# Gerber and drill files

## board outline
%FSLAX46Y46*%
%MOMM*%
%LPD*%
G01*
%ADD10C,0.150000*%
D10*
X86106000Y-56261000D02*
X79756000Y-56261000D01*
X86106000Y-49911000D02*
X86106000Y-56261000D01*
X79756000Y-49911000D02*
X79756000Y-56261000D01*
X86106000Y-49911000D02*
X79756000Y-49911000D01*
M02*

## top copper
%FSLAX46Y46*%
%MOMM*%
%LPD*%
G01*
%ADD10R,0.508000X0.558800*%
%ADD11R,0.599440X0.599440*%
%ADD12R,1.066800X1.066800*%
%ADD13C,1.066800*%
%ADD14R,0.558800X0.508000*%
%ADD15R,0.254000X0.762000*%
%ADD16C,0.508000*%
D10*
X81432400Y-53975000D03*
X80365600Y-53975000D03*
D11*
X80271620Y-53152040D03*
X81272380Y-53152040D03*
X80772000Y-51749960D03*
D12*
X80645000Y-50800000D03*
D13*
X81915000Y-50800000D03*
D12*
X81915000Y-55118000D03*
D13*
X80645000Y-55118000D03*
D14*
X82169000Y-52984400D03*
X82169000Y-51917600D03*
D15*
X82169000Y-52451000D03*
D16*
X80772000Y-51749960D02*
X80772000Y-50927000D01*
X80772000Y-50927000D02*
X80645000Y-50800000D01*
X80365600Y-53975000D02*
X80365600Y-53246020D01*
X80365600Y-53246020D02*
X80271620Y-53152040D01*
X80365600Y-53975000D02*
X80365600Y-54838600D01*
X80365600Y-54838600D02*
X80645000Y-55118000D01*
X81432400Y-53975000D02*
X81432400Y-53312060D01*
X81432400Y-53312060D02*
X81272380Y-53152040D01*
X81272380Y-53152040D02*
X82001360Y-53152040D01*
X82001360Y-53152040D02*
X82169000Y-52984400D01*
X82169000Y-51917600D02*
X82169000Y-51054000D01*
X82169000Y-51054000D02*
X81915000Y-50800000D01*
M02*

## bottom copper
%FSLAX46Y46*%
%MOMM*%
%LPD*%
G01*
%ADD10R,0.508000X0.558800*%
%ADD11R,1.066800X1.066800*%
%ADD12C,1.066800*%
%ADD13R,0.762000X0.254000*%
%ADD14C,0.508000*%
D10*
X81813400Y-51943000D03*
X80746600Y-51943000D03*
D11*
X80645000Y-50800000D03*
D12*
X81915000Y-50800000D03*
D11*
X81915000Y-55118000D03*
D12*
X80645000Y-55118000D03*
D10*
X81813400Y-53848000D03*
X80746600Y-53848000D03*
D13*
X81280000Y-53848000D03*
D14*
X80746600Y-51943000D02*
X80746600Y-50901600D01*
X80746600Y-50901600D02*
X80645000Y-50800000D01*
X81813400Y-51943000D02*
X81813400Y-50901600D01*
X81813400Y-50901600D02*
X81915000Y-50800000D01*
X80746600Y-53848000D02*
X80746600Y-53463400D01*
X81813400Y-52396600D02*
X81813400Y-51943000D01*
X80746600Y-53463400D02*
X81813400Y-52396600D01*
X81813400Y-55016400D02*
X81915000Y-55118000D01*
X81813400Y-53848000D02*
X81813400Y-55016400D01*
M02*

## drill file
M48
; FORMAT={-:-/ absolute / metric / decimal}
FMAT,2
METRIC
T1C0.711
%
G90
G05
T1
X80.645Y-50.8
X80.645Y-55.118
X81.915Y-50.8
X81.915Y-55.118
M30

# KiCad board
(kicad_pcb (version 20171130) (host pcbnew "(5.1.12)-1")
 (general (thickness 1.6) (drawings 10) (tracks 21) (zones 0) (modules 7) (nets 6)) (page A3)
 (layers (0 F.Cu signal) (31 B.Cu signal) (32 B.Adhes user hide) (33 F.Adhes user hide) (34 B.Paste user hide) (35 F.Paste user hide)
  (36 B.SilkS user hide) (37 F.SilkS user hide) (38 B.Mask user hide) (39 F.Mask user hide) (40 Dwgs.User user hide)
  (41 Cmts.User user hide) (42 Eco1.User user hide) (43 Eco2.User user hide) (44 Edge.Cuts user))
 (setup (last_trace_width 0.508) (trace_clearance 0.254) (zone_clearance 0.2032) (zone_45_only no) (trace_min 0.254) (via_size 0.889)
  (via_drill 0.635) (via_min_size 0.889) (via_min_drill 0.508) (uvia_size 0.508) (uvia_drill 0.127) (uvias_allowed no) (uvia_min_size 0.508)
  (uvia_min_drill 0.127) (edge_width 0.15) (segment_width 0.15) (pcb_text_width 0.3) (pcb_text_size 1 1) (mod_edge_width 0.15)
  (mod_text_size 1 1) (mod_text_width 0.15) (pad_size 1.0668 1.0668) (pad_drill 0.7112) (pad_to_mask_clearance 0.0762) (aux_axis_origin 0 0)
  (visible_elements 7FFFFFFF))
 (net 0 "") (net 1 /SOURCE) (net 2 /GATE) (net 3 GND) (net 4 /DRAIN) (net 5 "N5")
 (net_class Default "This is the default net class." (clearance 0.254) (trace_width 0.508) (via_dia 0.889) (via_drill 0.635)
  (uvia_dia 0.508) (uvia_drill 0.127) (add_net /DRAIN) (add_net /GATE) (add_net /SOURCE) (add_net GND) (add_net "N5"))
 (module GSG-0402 (layer F.Cu) (at 80.899 53.975) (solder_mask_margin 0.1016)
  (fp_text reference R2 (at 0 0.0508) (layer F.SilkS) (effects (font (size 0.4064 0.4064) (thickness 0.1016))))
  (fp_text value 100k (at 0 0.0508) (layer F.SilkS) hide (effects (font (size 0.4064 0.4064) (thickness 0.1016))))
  (pad 2 smd rect (at 0.5334 0) (size 0.508 0.5588) (layers F.Cu F.Paste F.Mask) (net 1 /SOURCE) (solder_mask_margin 0.1016))
  (pad 1 smd rect (at -0.5334 0) (size 0.508 0.5588) (layers F.Cu F.Paste F.Mask) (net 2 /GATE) (die_length -1518.485687)
   (solder_mask_margin 0.1016)))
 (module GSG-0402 (layer B.Cu) (at 81.28 51.943) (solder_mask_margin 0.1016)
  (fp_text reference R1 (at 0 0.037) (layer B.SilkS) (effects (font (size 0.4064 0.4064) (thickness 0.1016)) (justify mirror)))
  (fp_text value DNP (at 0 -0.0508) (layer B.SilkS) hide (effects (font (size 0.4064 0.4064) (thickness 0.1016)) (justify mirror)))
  (pad 2 smd rect (at 0.5334 0) (size 0.508 0.5588) (layers B.Cu B.Paste B.Mask) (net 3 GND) (solder_mask_margin 0.1016))
  (pad 1 smd rect (at -0.5334 0) (size 0.508 0.5588) (layers B.Cu B.Paste B.Mask) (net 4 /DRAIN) (die_length -1518.485687)
   (solder_mask_margin 0.1016)))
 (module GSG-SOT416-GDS (layer F.Cu) (at 80.772 52.451)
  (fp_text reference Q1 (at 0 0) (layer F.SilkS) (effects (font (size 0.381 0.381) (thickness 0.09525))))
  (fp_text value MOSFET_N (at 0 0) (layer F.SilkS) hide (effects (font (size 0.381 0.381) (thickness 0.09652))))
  (pad G smd rect (at -0.50038 0.70104) (size 0.59944 0.59944) (layers F.Cu F.Paste F.Mask) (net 2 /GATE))
  (pad S smd rect (at 0.50038 0.70104) (size 0.59944 0.59944) (layers F.Cu F.Paste F.Mask) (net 1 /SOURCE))
  (pad D smd rect (at 0 -0.70104) (size 0.59944 0.59944) (layers F.Cu F.Paste F.Mask) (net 4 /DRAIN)))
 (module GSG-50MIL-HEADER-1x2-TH (layer F.Cu) (at 81.28 50.8)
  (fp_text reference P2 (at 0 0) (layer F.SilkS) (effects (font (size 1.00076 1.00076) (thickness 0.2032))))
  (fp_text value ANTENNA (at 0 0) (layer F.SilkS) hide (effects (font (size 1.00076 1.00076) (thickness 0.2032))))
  (pad 1 thru_hole rect (at -0.635 0) (size 1.0668 1.0668) (drill 0.7112) (layers *.Cu *.Mask) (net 4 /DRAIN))
  (pad 2 thru_hole circle (at 0.635 0) (size 1.0668 1.0668) (drill 0.7112) (layers *.Cu *.Mask) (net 3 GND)))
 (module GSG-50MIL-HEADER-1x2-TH (layer F.Cu) (at 81.28 55.118 180)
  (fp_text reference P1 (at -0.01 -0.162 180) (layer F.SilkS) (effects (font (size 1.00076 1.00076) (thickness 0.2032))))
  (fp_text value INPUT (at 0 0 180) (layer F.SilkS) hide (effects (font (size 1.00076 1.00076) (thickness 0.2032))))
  (pad 1 thru_hole rect (at -0.635 0 180) (size 1.0668 1.0668) (drill 0.7112) (layers *.Cu *.Mask) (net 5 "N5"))
  (pad 2 thru_hole circle (at 0.635 0 180) (size 1.0668 1.0668) (drill 0.7112) (layers *.Cu *.Mask) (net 2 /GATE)))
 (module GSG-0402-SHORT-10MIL (layer B.Cu) (at 81.28 53.848) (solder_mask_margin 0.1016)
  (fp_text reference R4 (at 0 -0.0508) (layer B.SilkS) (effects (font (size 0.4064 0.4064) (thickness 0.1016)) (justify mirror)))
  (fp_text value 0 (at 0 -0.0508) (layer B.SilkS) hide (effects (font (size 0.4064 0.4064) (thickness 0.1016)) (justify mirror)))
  (pad 2 smd rect (at 0.5334 0) (size 0.508 0.5588) (layers B.Cu B.Mask) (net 5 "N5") (solder_mask_margin 0.1016))
  (pad 1 smd rect (at -0.5334 0) (size 0.508 0.5588) (layers B.Cu B.Mask) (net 3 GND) (die_length -1518.485687) (solder_mask_margin 0.1016))
  (pad "" smd rect (at 0 0) (size 0.762 0.254) (layers B.Cu B.Mask)))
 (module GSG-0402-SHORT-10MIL (layer F.Cu) (at 82.169 52.451 270) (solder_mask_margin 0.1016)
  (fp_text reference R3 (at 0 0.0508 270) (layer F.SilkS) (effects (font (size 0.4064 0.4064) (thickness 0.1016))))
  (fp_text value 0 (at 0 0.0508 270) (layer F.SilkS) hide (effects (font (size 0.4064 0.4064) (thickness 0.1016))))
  (pad 2 smd rect (at 0.5334 0 270) (size 0.508 0.5588) (layers F.Cu F.Mask) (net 1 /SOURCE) (solder_mask_margin 0.1016))
  (pad 1 smd rect (at -0.5334 0 270) (size 0.508 0.5588) (layers F.Cu F.Mask) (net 3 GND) (die_length -1518.485687)
   (solder_mask_margin 0.1016))
  (pad "" smd rect (at 0 0 270) (size 0.762 0.254) (layers F.Cu F.Mask)))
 (gr_line (start 86.106 56.261) (end 79.756 56.261) (angle 90) (layer Edge.Cuts) (width 0.15))
 (gr_line (start 86.106 49.911) (end 86.106 56.261) (angle 90) (layer Edge.Cuts) (width 0.15))
 (gr_line (start 79.756 49.911) (end 79.756 56.261) (angle 90) (layer Edge.Cuts) (width 0.15))
 (gr_line (start 86.106 49.911) (end 79.756 49.911) (angle 90) (layer Edge.Cuts) (width 0.15))
 (segment (start 80.7466 51.943) (end 80.7466 50.9016) (width 0.508) (layer B.Cu) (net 4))
 (segment (start 80.7466 50.9016) (end 80.645 50.8) (width 0.508) (layer B.Cu) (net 4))
 (segment (start 80.772 51.74996) (end 80.772 50.927) (width 0.508) (layer F.Cu) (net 4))
 (segment (start 80.772 50.927) (end 80.645 50.8) (width 0.508) (layer F.Cu) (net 4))
 (segment (start 80.3656 53.975) (end 80.3656 53.24602) (width 0.508) (layer F.Cu) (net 2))
 (segment (start 80.3656 53.24602) (end 80.27162 53.15204) (width 0.508) (layer F.Cu) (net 2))
 (segment (start 80.3656 53.975) (end 80.3656 54.8386) (width 0.508) (layer F.Cu) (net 2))
 (segment (start 80.3656 54.8386) (end 80.645 55.118) (width 0.508) (layer F.Cu) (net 2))
 (segment (start 81.4324 53.975) (end 81.4324 53.31206) (width 0.508) (layer F.Cu) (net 1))
 (segment (start 81.4324 53.31206) (end 81.27238 53.15204) (width 0.508) (layer F.Cu) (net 1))
 (segment (start 81.27238 53.15204) (end 82.00136 53.15204) (width 0.508) (layer F.Cu) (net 1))
 (segment (start 82.00136 53.15204) (end 82.169 52.9844) (width 0.508) (layer F.Cu) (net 1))
 (segment (start 81.8134 51.943) (end 81.8134 50.9016) (width 0.508) (layer B.Cu) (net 3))
 (segment (start 81.8134 50.9016) (end 81.915 50.8) (width 0.508) (layer B.Cu) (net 3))
 (segment (start 80.7466 53.848) (end 80.7466 53.4634) (width 0.508) (layer B.Cu) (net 3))
 (segment (start 81.8134 52.3966) (end 81.8134 51.943) (width 0.508) (layer B.Cu) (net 3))
 (segment (start 80.7466 53.4634) (end 81.8134 52.3966) (width 0.508) (layer B.Cu) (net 3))
 (segment (start 82.169 51.9176) (end 82.169 51.054) (width 0.508) (layer F.Cu) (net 3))
 (segment (start 82.169 51.054) (end 81.915 50.8) (width 0.508) (layer F.Cu) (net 3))
 (segment (start 81.8134 55.0164) (end 81.915 55.118) (width 0.508) (layer B.Cu) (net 5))
 (segment (start 81.8134 53.848) (end 81.8134 55.0164) (width 0.508) (layer B.Cu) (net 5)))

